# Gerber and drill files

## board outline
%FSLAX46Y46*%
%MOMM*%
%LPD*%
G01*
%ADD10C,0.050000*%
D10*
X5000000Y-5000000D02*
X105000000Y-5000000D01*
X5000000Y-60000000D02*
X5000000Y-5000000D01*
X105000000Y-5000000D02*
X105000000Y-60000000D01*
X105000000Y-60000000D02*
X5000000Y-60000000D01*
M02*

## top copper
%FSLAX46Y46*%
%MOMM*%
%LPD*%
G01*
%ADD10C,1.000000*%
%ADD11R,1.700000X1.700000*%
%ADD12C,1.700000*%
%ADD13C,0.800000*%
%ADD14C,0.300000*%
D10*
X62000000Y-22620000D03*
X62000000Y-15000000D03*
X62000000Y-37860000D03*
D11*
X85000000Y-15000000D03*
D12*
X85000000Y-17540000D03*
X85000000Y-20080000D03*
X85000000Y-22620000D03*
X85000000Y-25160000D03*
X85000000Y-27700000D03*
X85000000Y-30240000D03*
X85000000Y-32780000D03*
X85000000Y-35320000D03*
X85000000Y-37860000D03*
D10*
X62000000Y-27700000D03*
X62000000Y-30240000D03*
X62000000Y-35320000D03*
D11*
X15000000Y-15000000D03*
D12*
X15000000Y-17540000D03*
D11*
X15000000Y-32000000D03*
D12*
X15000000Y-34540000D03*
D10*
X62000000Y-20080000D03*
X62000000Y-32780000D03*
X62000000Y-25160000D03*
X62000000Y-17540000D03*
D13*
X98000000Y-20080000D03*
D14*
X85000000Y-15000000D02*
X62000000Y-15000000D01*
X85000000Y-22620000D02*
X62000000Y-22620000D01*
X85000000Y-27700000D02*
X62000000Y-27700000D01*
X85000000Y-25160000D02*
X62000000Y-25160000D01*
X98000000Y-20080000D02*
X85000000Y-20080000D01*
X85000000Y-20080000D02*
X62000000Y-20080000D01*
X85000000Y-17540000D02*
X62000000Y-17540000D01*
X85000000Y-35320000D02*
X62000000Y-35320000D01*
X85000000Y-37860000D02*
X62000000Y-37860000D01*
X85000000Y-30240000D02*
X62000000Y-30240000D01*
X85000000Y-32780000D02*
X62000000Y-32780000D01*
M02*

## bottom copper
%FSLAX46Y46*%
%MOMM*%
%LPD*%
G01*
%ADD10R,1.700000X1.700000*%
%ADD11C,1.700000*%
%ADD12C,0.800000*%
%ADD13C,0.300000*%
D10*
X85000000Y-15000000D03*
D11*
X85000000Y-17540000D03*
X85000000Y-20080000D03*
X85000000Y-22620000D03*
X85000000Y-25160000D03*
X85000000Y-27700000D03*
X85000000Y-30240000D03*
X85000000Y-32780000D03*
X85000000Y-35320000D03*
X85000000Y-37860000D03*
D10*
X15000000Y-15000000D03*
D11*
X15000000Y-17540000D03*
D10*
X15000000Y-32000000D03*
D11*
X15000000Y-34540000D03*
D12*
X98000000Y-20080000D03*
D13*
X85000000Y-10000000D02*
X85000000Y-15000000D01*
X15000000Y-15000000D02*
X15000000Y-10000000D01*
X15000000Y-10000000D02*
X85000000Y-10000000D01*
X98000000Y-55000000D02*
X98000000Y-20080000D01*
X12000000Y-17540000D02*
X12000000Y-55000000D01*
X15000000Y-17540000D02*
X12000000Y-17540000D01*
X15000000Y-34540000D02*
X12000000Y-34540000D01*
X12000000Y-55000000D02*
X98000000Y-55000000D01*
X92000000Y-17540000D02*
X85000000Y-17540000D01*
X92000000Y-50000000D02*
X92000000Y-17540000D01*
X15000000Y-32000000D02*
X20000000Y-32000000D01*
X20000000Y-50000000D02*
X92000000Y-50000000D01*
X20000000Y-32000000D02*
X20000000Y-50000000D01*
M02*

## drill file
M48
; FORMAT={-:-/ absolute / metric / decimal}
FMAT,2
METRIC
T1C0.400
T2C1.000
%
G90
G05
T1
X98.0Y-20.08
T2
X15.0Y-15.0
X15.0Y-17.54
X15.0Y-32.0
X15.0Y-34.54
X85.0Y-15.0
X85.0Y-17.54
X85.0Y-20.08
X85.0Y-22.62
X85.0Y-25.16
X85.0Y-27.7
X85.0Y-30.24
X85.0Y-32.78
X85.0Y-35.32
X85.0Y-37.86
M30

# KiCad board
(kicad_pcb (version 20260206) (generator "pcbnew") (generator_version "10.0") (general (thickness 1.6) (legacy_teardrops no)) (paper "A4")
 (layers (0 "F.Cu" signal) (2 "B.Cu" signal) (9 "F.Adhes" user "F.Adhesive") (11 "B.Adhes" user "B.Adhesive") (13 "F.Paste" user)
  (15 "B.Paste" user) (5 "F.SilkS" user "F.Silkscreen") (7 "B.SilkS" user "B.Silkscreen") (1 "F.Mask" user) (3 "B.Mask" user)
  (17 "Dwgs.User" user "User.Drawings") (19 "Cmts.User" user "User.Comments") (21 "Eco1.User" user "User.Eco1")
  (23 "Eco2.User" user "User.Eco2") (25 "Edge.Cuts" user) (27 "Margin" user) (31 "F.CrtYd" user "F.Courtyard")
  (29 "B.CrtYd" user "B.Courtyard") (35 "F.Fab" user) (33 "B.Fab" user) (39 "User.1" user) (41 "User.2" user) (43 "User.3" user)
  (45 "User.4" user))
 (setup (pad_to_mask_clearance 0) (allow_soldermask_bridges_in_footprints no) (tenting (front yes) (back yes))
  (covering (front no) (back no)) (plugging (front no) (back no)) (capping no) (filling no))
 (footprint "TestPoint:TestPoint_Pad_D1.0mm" (layer "F.Cu") (at 62 22.62)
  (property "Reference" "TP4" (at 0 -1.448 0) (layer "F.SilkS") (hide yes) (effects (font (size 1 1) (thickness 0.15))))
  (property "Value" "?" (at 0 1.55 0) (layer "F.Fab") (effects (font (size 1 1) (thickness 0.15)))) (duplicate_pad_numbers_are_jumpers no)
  (pad "1" smd circle (at 0 0) (size 1 1) (layers "F.Cu" "F.Mask") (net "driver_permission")))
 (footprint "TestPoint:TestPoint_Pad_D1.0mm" (layer "F.Cu") (at 62 15)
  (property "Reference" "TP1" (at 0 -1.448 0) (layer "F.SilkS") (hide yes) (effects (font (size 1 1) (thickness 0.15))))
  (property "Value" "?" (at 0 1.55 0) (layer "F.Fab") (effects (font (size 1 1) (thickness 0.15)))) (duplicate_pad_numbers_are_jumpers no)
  (pad "1" smd circle (at 0 0) (size 1 1) (layers "F.Cu" "F.Mask") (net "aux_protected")))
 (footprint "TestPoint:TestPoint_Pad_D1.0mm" (layer "F.Cu") (at 62 37.86)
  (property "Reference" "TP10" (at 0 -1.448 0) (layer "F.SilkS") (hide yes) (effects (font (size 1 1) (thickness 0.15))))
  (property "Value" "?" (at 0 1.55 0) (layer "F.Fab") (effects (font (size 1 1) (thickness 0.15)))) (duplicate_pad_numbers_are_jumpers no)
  (pad "1" smd circle (at 0 0) (size 1 1) (layers "F.Cu" "F.Mask") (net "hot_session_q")))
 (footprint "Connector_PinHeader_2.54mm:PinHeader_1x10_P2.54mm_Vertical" (layer "F.Cu") (at 85 15)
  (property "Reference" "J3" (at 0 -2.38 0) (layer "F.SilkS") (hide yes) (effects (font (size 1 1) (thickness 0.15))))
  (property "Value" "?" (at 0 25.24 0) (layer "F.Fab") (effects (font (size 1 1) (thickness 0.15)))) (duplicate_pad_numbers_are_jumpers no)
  (pad "1" thru_hole rect (at 0 0) (size 1.7 1.7) (drill 1) (layers "*.Cu" "*.Mask") (remove_unused_layers no) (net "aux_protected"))
  (pad "2" thru_hole circle (at 0 2.54) (size 1.7 1.7) (drill 1) (layers "*.Cu" "*.Mask") (remove_unused_layers no) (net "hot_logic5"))
  (pad "3" thru_hole circle (at 0 5.08) (size 1.7 1.7) (drill 1) (layers "*.Cu" "*.Mask") (remove_unused_layers no) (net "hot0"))
  (pad "4" thru_hole circle (at 0 7.62) (size 1.7 1.7) (drill 1) (layers "*.Cu" "*.Mask") (remove_unused_layers no)
   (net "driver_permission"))
  (pad "5" thru_hole circle (at 0 10.16) (size 1.7 1.7) (drill 1) (layers "*.Cu" "*.Mask") (remove_unused_layers no) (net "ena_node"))
  (pad "6" thru_hole circle (at 0 12.7) (size 1.7 1.7) (drill 1) (layers "*.Cu" "*.Mask") (remove_unused_layers no) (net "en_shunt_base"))
  (pad "7" thru_hole circle (at 0 15.24) (size 1.7 1.7) (drill 1) (layers "*.Cu" "*.Mask") (remove_unused_layers no) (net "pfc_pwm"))
  (pad "8" thru_hole circle (at 0 17.78) (size 1.7 1.7) (drill 1) (layers "*.Cu" "*.Mask") (remove_unused_layers no) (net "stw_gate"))
  (pad "9" thru_hole circle (at 0 20.32) (size 1.7 1.7) (drill 1) (layers "*.Cu" "*.Mask") (remove_unused_layers no) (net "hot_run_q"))
  (pad "10" thru_hole circle (at 0 22.86) (size 1.7 1.7) (drill 1) (layers "*.Cu" "*.Mask") (remove_unused_layers no) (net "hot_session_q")))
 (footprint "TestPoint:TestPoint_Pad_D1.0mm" (layer "F.Cu") (at 62 27.7)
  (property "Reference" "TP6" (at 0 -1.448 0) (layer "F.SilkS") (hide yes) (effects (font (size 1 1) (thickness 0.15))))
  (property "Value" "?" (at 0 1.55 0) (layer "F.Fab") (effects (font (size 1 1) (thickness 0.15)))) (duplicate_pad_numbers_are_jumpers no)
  (pad "1" smd circle (at 0 0) (size 1 1) (layers "F.Cu" "F.Mask") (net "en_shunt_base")))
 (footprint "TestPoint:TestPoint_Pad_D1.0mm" (layer "F.Cu") (at 62 30.24)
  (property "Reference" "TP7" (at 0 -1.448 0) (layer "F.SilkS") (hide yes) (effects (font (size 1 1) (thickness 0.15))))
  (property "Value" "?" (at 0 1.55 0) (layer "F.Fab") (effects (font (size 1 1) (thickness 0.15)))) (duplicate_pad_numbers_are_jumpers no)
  (pad "1" smd circle (at 0 0) (size 1 1) (layers "F.Cu" "F.Mask") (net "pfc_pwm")))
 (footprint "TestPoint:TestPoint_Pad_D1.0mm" (layer "F.Cu") (at 62 35.32)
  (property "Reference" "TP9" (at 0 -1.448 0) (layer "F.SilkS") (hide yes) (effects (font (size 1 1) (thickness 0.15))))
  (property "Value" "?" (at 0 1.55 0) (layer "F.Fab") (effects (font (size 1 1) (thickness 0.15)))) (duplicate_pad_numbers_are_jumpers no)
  (pad "1" smd circle (at 0 0) (size 1 1) (layers "F.Cu" "F.Mask") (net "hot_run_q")))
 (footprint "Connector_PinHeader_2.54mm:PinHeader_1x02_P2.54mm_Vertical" (layer "F.Cu") (at 15 15)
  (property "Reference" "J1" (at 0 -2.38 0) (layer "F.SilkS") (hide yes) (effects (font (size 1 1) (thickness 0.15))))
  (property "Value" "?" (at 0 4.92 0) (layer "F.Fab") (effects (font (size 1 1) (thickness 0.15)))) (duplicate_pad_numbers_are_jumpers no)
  (pad "1" thru_hole rect (at 0 0) (size 1.7 1.7) (drill 1) (layers "*.Cu" "*.Mask") (remove_unused_layers no) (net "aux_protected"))
  (pad "2" thru_hole circle (at 0 2.54) (size 1.7 1.7) (drill 1) (layers "*.Cu" "*.Mask") (remove_unused_layers no) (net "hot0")))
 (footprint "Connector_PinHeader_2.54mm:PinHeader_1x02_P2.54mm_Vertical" (layer "F.Cu") (at 15 32)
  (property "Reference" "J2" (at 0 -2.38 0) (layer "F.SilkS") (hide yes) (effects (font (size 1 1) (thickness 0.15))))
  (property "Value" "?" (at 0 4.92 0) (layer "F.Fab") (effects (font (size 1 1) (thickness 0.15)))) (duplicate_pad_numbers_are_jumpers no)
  (pad "1" thru_hole rect (at 0 0) (size 1.7 1.7) (drill 1) (layers "*.Cu" "*.Mask") (remove_unused_layers no) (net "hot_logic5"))
  (pad "2" thru_hole circle (at 0 2.54) (size 1.7 1.7) (drill 1) (layers "*.Cu" "*.Mask") (remove_unused_layers no) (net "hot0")))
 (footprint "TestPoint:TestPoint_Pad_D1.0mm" (layer "F.Cu") (at 62 20.08)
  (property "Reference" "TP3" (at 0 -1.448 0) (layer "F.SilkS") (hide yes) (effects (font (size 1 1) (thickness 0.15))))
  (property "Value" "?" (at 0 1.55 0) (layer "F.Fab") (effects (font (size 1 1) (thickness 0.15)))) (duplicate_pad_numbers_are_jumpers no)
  (pad "1" smd circle (at 0 0) (size 1 1) (layers "F.Cu" "F.Mask") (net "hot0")))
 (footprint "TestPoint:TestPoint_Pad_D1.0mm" (layer "F.Cu") (at 62 32.78)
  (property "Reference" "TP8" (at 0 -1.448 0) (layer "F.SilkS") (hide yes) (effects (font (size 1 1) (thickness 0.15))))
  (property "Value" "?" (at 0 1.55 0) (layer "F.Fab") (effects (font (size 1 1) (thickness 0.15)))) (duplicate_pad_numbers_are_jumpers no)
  (pad "1" smd circle (at 0 0) (size 1 1) (layers "F.Cu" "F.Mask") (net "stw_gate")))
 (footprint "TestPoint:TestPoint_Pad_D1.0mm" (layer "F.Cu") (at 62 25.16)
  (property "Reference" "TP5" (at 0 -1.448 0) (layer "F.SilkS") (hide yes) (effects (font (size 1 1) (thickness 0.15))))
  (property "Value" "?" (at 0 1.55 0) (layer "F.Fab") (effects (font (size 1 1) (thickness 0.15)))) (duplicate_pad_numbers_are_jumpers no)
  (pad "1" smd circle (at 0 0) (size 1 1) (layers "F.Cu" "F.Mask") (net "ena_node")))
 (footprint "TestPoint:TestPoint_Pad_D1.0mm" (layer "F.Cu") (at 62 17.54)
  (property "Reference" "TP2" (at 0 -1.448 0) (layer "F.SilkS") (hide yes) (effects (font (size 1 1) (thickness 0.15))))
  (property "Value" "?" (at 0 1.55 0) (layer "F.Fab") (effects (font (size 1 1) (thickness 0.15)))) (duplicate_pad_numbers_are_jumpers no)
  (pad "1" smd circle (at 0 0) (size 1 1) (layers "F.Cu" "F.Mask") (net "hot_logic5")))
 (gr_line (start 5 5) (end 105 5) (stroke (width 0.05) (type default)) (layer "Edge.Cuts"))
 (gr_line (start 5 60) (end 5 5) (stroke (width 0.05) (type default)) (layer "Edge.Cuts"))
 (gr_line (start 105 5) (end 105 60) (stroke (width 0.05) (type default)) (layer "Edge.Cuts"))
 (gr_line (start 105 60) (end 5 60) (stroke (width 0.05) (type default)) (layer "Edge.Cuts"))
 (segment (start 85 15) (end 62 15) (width 0.3) (layer "F.Cu") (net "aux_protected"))
 (segment (start 85 10) (end 85 15) (width 0.3) (layer "B.Cu") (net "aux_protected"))
 (segment (start 15 15) (end 15 10) (width 0.3) (layer "B.Cu") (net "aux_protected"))
 (segment (start 15 10) (end 85 10) (width 0.3) (layer "B.Cu") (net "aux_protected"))
 (segment (start 85 22.62) (end 62 22.62) (width 0.3) (layer "F.Cu") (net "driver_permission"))
 (segment (start 85 27.7) (end 62 27.7) (width 0.3) (layer "F.Cu") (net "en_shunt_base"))
 (segment (start 85 25.16) (end 62 25.16) (width 0.3) (layer "F.Cu") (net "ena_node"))
 (segment (start 98 20.08) (end 85 20.08) (width 0.3) (layer "F.Cu") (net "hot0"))
 (segment (start 85 20.08) (end 62 20.08) (width 0.3) (layer "F.Cu") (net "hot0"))
 (via (at 98 20.08) (size 0.8) (drill 0.4) (layers "F.Cu" "B.Cu") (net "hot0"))
 (segment (start 98 55) (end 98 20.08) (width 0.3) (layer "B.Cu") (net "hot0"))
 (segment (start 12 17.54) (end 12 55) (width 0.3) (layer "B.Cu") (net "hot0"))
 (segment (start 15 17.54) (end 12 17.54) (width 0.3) (layer "B.Cu") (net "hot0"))
 (segment (start 15 34.54) (end 12 34.54) (width 0.3) (layer "B.Cu") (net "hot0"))
 (segment (start 12 55) (end 98 55) (width 0.3) (layer "B.Cu") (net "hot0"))
 (segment (start 85 17.54) (end 62 17.54) (width 0.3) (layer "F.Cu") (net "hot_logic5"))
 (segment (start 92 17.54) (end 85 17.54) (width 0.3) (layer "B.Cu") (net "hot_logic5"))
 (segment (start 92 50) (end 92 17.54) (width 0.3) (layer "B.Cu") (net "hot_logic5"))
 (segment (start 15 32) (end 20 32) (width 0.3) (layer "B.Cu") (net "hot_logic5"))
 (segment (start 20 50) (end 92 50) (width 0.3) (layer "B.Cu") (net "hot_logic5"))
 (segment (start 20 32) (end 20 50) (width 0.3) (layer "B.Cu") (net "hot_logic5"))
 (segment (start 85 35.32) (end 62 35.32) (width 0.3) (layer "F.Cu") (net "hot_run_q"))
 (segment (start 85 37.86) (end 62 37.86) (width 0.3) (layer "F.Cu") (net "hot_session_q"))
 (segment (start 85 30.24) (end 62 30.24) (width 0.3) (layer "F.Cu") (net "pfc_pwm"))
 (segment (start 85 32.78) (end 62 32.78) (width 0.3) (layer "F.Cu") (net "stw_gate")))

